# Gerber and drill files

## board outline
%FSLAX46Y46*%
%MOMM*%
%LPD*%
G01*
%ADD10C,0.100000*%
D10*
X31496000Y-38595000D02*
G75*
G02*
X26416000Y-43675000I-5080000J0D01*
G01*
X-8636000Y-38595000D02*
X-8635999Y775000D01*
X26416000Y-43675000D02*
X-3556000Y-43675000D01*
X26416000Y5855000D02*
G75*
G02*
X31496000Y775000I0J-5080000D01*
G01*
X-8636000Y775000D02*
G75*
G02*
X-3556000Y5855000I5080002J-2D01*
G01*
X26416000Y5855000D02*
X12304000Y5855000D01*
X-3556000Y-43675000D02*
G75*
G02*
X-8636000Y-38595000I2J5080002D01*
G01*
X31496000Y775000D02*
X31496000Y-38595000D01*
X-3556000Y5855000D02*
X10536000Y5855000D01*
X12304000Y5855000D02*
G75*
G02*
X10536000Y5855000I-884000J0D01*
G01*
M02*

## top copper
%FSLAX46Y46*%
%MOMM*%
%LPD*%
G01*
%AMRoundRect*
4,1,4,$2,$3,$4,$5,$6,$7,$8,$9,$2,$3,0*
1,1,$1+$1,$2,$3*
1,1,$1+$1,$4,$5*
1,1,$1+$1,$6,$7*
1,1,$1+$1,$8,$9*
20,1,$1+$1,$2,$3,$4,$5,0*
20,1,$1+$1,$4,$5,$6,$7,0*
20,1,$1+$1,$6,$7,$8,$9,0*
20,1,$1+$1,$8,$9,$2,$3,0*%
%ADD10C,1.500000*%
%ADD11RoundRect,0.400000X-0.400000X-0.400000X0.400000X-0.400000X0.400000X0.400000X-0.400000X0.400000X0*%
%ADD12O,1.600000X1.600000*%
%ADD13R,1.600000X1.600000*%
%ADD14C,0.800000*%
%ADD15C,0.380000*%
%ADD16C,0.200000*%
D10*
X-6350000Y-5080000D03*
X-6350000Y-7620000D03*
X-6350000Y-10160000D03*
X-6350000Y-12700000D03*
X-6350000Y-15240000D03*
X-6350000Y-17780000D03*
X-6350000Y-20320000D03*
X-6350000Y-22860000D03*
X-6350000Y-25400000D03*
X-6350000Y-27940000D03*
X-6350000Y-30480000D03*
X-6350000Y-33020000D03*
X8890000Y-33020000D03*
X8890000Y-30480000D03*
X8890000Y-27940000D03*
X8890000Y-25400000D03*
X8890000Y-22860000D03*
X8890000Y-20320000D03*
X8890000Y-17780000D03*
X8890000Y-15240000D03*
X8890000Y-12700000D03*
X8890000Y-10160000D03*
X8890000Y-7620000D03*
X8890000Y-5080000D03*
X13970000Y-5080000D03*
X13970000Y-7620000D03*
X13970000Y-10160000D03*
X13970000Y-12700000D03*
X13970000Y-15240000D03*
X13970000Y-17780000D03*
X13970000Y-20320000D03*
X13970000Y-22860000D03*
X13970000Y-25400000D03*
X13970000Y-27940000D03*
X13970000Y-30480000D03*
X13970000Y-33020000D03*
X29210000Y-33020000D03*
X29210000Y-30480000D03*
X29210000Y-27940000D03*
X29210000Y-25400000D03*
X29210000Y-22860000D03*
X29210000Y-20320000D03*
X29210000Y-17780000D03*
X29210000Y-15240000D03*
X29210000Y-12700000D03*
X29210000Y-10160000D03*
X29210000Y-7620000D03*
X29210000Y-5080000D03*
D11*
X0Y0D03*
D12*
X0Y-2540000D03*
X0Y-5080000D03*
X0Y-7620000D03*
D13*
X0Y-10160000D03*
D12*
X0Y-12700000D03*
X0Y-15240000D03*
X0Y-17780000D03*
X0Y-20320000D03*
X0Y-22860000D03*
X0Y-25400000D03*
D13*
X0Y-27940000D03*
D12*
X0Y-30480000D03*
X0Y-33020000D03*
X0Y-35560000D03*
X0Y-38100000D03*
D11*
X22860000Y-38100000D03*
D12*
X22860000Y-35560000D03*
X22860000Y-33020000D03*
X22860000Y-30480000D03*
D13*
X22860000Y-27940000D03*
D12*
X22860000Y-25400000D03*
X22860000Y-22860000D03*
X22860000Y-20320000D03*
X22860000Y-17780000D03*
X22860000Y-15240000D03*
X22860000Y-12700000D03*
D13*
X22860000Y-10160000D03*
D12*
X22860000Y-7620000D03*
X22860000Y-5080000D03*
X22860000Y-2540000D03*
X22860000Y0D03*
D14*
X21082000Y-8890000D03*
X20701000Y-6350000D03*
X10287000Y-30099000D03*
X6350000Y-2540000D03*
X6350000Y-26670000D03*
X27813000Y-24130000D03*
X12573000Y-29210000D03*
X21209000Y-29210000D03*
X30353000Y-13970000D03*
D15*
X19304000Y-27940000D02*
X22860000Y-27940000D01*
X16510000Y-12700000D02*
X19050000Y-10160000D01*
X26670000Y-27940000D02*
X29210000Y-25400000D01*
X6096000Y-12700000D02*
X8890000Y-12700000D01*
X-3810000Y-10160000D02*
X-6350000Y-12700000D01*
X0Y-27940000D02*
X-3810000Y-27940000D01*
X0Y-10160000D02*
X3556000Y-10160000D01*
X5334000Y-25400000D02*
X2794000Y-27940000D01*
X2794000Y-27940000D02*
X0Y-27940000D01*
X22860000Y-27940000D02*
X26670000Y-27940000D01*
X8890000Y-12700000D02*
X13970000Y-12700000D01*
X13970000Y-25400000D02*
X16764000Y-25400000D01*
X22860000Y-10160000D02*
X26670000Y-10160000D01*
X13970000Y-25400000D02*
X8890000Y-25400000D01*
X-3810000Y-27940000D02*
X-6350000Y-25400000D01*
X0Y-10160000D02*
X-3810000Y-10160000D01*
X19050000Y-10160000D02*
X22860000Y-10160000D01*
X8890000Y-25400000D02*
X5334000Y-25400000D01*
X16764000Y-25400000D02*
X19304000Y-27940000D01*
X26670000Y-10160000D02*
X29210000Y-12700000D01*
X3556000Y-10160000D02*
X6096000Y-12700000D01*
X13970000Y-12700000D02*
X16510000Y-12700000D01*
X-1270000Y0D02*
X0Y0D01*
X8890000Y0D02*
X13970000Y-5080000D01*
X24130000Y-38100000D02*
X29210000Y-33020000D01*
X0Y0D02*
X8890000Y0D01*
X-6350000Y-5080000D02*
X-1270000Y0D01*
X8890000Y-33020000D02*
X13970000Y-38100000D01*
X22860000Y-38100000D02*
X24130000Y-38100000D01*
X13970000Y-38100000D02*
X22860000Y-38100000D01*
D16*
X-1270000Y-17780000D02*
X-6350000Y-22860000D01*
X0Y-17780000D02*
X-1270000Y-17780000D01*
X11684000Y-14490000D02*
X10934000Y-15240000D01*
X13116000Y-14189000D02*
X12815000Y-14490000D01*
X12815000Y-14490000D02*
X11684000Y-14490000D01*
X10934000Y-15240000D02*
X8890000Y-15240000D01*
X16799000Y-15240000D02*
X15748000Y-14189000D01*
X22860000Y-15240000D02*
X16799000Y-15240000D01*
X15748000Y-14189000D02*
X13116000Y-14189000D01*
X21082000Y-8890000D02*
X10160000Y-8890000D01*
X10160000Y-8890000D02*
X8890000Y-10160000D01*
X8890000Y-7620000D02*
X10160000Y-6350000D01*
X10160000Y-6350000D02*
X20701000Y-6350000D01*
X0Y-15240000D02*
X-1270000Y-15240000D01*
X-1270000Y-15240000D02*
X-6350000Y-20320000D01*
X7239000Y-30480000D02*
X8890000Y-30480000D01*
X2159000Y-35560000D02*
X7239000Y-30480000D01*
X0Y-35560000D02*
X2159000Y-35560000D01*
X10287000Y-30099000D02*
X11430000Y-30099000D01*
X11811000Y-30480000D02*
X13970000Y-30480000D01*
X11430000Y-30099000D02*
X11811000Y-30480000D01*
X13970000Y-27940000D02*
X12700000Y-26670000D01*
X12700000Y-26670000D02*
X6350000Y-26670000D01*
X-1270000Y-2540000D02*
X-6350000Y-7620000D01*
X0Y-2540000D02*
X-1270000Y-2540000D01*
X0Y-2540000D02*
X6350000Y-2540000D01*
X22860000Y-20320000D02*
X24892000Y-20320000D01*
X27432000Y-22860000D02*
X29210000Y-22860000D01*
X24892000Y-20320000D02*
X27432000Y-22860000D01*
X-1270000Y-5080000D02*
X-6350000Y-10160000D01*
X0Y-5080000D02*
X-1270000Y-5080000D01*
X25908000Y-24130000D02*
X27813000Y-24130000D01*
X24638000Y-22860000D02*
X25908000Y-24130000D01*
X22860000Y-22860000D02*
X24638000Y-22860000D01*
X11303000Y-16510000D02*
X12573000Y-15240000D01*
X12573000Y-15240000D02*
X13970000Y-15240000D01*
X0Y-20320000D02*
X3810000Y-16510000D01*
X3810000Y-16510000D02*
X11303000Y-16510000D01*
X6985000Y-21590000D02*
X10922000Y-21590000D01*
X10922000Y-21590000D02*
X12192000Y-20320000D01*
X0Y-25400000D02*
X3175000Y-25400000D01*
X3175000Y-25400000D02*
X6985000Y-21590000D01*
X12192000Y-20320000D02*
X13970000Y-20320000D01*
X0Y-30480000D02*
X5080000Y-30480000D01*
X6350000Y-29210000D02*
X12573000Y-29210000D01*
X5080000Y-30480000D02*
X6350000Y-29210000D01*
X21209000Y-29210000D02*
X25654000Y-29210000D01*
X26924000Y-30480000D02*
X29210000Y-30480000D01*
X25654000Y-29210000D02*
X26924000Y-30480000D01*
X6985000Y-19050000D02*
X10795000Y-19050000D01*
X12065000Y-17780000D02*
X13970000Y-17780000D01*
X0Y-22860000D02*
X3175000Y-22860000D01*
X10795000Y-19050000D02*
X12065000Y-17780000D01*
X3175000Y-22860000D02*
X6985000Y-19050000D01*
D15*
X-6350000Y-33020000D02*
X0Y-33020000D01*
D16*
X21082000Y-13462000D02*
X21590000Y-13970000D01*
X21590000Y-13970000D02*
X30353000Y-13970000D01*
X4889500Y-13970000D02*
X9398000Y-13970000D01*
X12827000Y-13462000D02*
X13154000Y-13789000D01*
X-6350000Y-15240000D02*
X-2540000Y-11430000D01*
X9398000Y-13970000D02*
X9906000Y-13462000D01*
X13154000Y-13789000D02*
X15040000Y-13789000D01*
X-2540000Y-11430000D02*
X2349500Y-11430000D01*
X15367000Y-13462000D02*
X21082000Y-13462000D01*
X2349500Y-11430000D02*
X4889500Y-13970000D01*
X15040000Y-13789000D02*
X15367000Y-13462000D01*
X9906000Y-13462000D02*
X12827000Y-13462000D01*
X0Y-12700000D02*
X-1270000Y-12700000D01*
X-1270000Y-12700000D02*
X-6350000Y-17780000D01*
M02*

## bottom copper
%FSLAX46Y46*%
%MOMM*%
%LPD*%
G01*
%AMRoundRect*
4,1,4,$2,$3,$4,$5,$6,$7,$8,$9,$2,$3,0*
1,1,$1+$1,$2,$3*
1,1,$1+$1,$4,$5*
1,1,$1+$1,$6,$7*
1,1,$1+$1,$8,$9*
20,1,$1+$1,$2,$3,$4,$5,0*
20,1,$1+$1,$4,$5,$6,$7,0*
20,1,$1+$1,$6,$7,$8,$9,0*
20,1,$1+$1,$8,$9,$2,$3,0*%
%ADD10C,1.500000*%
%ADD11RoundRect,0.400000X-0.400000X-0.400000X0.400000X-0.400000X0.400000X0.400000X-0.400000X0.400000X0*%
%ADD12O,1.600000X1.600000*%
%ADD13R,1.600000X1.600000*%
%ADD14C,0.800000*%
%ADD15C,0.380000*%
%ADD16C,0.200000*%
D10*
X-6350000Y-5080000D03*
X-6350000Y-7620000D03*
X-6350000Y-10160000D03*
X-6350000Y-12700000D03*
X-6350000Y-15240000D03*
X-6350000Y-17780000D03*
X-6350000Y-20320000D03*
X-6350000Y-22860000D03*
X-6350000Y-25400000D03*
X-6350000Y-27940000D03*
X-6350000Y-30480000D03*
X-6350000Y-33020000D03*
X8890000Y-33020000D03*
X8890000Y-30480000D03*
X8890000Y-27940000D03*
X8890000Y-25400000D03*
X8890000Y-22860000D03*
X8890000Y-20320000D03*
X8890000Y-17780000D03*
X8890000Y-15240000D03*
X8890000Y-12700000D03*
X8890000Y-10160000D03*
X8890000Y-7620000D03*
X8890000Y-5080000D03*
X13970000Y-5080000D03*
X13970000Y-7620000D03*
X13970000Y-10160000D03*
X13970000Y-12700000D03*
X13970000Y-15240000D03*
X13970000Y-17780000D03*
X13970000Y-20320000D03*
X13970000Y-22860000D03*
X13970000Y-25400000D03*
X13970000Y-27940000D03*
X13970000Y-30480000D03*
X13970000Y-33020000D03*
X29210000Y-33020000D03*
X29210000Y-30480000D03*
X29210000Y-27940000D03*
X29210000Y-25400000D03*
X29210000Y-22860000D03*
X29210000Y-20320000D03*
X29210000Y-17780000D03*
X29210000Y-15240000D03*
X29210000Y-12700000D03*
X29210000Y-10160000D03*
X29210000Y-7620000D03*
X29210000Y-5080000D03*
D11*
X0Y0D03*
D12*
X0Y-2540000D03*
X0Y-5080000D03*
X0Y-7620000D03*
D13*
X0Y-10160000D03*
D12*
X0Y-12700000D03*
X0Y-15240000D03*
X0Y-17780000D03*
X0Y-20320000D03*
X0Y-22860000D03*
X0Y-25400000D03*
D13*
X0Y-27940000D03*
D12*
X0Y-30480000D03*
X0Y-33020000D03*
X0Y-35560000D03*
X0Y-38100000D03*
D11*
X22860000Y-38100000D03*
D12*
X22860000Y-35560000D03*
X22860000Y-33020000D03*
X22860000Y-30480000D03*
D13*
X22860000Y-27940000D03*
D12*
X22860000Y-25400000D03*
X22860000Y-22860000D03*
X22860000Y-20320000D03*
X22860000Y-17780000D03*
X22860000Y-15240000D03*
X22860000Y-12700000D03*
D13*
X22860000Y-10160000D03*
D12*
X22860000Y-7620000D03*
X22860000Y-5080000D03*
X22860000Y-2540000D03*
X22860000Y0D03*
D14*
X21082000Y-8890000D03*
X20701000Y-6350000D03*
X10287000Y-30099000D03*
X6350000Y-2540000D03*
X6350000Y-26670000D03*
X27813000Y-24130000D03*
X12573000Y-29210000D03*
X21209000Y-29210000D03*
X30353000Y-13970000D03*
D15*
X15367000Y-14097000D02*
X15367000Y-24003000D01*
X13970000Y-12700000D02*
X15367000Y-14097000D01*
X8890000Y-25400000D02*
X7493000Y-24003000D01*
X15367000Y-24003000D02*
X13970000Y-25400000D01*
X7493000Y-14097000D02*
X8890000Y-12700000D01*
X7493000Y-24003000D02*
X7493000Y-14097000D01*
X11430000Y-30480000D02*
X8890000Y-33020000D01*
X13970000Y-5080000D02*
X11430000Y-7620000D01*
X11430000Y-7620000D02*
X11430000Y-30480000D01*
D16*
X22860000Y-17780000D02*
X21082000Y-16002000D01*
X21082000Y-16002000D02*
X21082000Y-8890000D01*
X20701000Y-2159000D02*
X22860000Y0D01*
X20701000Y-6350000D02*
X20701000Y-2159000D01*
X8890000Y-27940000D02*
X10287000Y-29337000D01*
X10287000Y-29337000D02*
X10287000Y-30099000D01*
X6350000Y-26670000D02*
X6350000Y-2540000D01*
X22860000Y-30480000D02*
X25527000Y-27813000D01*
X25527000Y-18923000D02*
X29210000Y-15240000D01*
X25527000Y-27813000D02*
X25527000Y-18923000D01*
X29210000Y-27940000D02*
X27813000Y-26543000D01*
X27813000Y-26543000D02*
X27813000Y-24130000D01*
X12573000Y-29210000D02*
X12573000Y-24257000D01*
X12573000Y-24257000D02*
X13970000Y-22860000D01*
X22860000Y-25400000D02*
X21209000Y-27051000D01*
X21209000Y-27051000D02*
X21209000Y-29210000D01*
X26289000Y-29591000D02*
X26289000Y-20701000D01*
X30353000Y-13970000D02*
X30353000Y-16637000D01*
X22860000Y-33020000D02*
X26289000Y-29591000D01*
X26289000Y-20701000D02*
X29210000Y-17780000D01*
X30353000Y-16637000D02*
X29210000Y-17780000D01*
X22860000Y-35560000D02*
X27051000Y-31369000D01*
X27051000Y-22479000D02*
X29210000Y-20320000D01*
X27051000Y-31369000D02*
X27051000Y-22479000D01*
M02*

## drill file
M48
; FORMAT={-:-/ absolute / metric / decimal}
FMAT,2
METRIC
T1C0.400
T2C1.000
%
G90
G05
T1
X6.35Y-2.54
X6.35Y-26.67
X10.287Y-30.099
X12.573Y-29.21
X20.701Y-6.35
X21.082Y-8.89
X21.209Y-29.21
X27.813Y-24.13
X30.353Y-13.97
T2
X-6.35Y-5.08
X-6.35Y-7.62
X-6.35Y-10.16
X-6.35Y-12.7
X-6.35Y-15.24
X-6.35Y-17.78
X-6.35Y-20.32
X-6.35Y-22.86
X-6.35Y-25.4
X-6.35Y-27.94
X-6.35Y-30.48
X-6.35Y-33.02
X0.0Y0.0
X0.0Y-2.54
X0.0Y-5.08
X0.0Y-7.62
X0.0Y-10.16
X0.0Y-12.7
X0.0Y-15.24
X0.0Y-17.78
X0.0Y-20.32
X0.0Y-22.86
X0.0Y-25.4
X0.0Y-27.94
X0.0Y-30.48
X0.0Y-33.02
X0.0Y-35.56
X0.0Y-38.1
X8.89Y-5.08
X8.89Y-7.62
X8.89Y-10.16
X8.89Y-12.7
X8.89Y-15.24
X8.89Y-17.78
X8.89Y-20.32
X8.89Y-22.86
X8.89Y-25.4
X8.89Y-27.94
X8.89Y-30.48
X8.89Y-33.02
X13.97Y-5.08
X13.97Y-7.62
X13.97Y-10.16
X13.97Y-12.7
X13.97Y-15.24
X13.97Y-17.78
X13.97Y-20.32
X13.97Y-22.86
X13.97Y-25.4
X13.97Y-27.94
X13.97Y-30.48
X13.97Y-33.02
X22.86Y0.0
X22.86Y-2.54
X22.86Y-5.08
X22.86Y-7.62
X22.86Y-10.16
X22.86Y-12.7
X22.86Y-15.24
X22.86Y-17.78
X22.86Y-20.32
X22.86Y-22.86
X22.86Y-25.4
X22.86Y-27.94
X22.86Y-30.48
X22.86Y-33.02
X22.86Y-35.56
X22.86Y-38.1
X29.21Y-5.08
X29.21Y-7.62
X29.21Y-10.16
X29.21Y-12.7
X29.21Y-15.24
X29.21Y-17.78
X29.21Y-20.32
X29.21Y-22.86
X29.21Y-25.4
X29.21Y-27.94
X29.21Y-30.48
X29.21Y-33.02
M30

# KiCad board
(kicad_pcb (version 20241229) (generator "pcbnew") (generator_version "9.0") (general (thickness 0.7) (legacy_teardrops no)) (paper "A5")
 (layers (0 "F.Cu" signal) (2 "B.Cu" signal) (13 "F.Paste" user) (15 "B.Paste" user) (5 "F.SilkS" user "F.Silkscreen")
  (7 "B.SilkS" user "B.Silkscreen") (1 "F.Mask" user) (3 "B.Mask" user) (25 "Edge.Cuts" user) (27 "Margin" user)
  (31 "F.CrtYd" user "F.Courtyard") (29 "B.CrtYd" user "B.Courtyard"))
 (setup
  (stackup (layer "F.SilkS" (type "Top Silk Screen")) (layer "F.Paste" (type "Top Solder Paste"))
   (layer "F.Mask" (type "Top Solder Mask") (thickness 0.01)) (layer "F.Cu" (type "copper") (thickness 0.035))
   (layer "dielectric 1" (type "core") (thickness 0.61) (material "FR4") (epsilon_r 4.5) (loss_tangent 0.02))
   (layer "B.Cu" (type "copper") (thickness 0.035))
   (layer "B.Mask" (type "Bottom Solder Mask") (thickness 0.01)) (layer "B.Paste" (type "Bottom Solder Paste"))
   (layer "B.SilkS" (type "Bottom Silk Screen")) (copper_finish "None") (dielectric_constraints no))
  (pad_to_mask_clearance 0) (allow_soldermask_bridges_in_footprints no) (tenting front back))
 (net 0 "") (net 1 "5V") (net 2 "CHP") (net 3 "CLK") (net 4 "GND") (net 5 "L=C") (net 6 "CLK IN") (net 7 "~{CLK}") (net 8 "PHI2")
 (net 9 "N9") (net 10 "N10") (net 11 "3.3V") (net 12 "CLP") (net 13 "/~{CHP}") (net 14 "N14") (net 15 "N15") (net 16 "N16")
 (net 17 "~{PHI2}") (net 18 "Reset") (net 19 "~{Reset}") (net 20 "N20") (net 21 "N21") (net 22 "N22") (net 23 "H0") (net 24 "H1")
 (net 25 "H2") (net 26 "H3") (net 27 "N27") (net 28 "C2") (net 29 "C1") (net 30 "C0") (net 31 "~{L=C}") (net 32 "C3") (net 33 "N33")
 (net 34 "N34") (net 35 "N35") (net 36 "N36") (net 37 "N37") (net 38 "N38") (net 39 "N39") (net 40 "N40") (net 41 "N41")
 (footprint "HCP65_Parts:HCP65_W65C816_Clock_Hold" (layer "F.Cu") (at -6.35 5.08)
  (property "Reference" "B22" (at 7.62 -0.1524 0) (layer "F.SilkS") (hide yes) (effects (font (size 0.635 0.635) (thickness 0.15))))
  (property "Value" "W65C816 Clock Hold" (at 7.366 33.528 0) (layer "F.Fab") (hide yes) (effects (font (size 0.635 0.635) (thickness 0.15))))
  (pad "1" thru_hole circle (at 0 0) (size 1.5 1.5) (drill 1) (layers "*.Cu" "*.Mask") (remove_unused_layers no) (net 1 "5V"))
  (pad "2" thru_hole circle (at 0 2.54) (size 1.5 1.5) (drill 1) (layers "*.Cu" "*.Mask") (remove_unused_layers no) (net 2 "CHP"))
  (pad "3" thru_hole circle (at 0 5.08) (size 1.5 1.5) (drill 1) (layers "*.Cu" "*.Mask") (remove_unused_layers no) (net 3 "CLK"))
  (pad "4" thru_hole circle (at 0 7.62) (size 1.5 1.5) (drill 1) (layers "*.Cu" "*.Mask") (remove_unused_layers no) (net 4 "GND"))
  (pad "5" thru_hole circle (at 0 10.16) (size 1.5 1.5) (drill 1) (layers "*.Cu" "*.Mask") (remove_unused_layers no) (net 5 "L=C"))
  (pad "6" thru_hole circle (at 0 12.7) (size 1.5 1.5) (drill 1) (layers "*.Cu" "*.Mask") (remove_unused_layers no) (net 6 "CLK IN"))
  (pad "7" thru_hole circle (at 0 15.24) (size 1.5 1.5) (drill 1) (layers "*.Cu" "*.Mask") (remove_unused_layers no) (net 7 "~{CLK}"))
  (pad "8" thru_hole circle (at 0 17.78) (size 1.5 1.5) (drill 1) (layers "*.Cu" "*.Mask") (remove_unused_layers no) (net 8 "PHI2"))
  (pad "9" thru_hole circle (at 0 20.32) (size 1.5 1.5) (drill 1) (layers "*.Cu" "*.Mask") (remove_unused_layers no) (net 4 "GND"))
  (pad "10" thru_hole circle (at 0 22.86) (size 1.5 1.5) (drill 1) (layers "*.Cu" "*.Mask") (remove_unused_layers no) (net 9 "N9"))
  (pad "11" thru_hole circle (at 0 25.4) (size 1.5 1.5) (drill 1) (layers "*.Cu" "*.Mask") (remove_unused_layers no) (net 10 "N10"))
  (pad "12" thru_hole circle (at 0 27.94) (size 1.5 1.5) (drill 1) (layers "*.Cu" "*.Mask") (remove_unused_layers no) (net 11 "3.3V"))
  (pad "13" thru_hole circle (at 15.24 27.94) (size 1.5 1.5) (drill 1) (layers "*.Cu" "*.Mask") (remove_unused_layers no) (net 1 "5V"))
  (pad "14" thru_hole circle (at 15.24 25.4) (size 1.5 1.5) (drill 1) (layers "*.Cu" "*.Mask") (remove_unused_layers no) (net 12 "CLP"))
  (pad "15" thru_hole circle (at 15.24 22.86) (size 1.5 1.5) (drill 1) (layers "*.Cu" "*.Mask") (remove_unused_layers no) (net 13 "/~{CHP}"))
  (pad "16" thru_hole circle (at 15.24 20.32) (size 1.5 1.5) (drill 1) (layers "*.Cu" "*.Mask") (remove_unused_layers no) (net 4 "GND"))
  (pad "17" thru_hole circle (at 15.24 17.78) (size 1.5 1.5) (drill 1) (layers "*.Cu" "*.Mask") (remove_unused_layers no) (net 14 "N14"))
  (pad "18" thru_hole circle (at 15.24 15.24) (size 1.5 1.5) (drill 1) (layers "*.Cu" "*.Mask") (remove_unused_layers no) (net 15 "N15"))
  (pad "19" thru_hole circle (at 15.24 12.7) (size 1.5 1.5) (drill 1) (layers "*.Cu" "*.Mask") (remove_unused_layers no) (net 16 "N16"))
  (pad "20" thru_hole circle (at 15.24 10.16) (size 1.5 1.5) (drill 1) (layers "*.Cu" "*.Mask") (remove_unused_layers no) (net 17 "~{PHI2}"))
  (pad "21" thru_hole circle (at 15.24 7.62) (size 1.5 1.5) (drill 1) (layers "*.Cu" "*.Mask") (remove_unused_layers no) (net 4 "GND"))
  (pad "22" thru_hole circle (at 15.24 5.08) (size 1.5 1.5) (drill 1) (layers "*.Cu" "*.Mask") (remove_unused_layers no) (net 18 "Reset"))
  (pad "23" thru_hole circle (at 15.24 2.54) (size 1.5 1.5) (drill 1) (layers "*.Cu" "*.Mask") (remove_unused_layers no) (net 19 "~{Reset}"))
  (pad "24" thru_hole circle (at 15.24 0) (size 1.5 1.5) (drill 1) (layers "*.Cu" "*.Mask") (remove_unused_layers no) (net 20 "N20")))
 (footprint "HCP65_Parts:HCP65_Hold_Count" (layer "F.Cu") (at 13.97 5.08)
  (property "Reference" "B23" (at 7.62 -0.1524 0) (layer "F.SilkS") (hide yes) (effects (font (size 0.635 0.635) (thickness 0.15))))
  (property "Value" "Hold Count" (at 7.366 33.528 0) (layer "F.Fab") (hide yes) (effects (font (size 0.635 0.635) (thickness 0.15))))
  (pad "1" thru_hole circle (at 0 0) (size 1.5 1.5) (drill 1) (layers "*.Cu" "*.Mask") (remove_unused_layers no) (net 1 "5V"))
  (pad "2" thru_hole circle (at 0 2.54) (size 1.5 1.5) (drill 1) (layers "*.Cu" "*.Mask") (remove_unused_layers no) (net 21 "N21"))
  (pad "3" thru_hole circle (at 0 5.08) (size 1.5 1.5) (drill 1) (layers "*.Cu" "*.Mask") (remove_unused_layers no) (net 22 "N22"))
  (pad "4" thru_hole circle (at 0 7.62) (size 1.5 1.5) (drill 1) (layers "*.Cu" "*.Mask") (remove_unused_layers no) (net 4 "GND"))
  (pad "5" thru_hole circle (at 0 10.16) (size 1.5 1.5) (drill 1) (layers "*.Cu" "*.Mask") (remove_unused_layers no) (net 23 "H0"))
  (pad "6" thru_hole circle (at 0 12.7) (size 1.5 1.5) (drill 1) (layers "*.Cu" "*.Mask") (remove_unused_layers no) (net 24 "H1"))
  (pad "7" thru_hole circle (at 0 15.24) (size 1.5 1.5) (drill 1) (layers "*.Cu" "*.Mask") (remove_unused_layers no) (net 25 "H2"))
  (pad "8" thru_hole circle (at 0 17.78) (size 1.5 1.5) (drill 1) (layers "*.Cu" "*.Mask") (remove_unused_layers no) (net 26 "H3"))
  (pad "9" thru_hole circle (at 0 20.32) (size 1.5 1.5) (drill 1) (layers "*.Cu" "*.Mask") (remove_unused_layers no) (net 4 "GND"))
  (pad "10" thru_hole circle (at 0 22.86) (size 1.5 1.5) (drill 1) (layers "*.Cu" "*.Mask") (remove_unused_layers no) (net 2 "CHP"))
  (pad "11" thru_hole circle (at 0 25.4) (size 1.5 1.5) (drill 1) (layers "*.Cu" "*.Mask") (remove_unused_layers no) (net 13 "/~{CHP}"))
  (pad "12" thru_hole circle (at 0 27.94) (size 1.5 1.5) (drill 1) (layers "*.Cu" "*.Mask") (remove_unused_layers no) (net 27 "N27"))
  (pad "13" thru_hole circle (at 15.24 27.94) (size 1.5 1.5) (drill 1) (layers "*.Cu" "*.Mask") (remove_unused_layers no) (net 1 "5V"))
  (pad "14" thru_hole circle (at 15.24 25.4) (size 1.5 1.5) (drill 1) (layers "*.Cu" "*.Mask") (remove_unused_layers no) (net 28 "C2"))
  (pad "15" thru_hole circle (at 15.24 22.86) (size 1.5 1.5) (drill 1) (layers "*.Cu" "*.Mask") (remove_unused_layers no) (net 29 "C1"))
  (pad "16" thru_hole circle (at 15.24 20.32) (size 1.5 1.5) (drill 1) (layers "*.Cu" "*.Mask") (remove_unused_layers no) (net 4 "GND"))
  (pad "17" thru_hole circle (at 15.24 17.78) (size 1.5 1.5) (drill 1) (layers "*.Cu" "*.Mask") (remove_unused_layers no) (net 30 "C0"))
  (pad "18" thru_hole circle (at 15.24 15.24) (size 1.5 1.5) (drill 1) (layers "*.Cu" "*.Mask") (remove_unused_layers no) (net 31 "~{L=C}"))
  (pad "19" thru_hole circle (at 15.24 12.7) (size 1.5 1.5) (drill 1) (layers "*.Cu" "*.Mask") (remove_unused_layers no) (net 5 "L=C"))
  (pad "20" thru_hole circle (at 15.24 10.16) (size 1.5 1.5) (drill 1) (layers "*.Cu" "*.Mask") (remove_unused_layers no) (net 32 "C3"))
  (pad "21" thru_hole circle (at 15.24 7.62) (size 1.5 1.5) (drill 1) (layers "*.Cu" "*.Mask") (remove_unused_layers no) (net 4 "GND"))
  (pad "22" thru_hole circle (at 15.24 5.08) (size 1.5 1.5) (drill 1) (layers "*.Cu" "*.Mask") (remove_unused_layers no) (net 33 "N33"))
  (pad "23" thru_hole circle (at 15.24 2.54) (size 1.5 1.5) (drill 1) (layers "*.Cu" "*.Mask") (remove_unused_layers no) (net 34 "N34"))
  (pad "24" thru_hole circle (at 15.24 0) (size 1.5 1.5) (drill 1) (layers "*.Cu" "*.Mask") (remove_unused_layers no) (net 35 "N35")))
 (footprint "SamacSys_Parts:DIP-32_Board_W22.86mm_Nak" (layer "F.Cu") (at 0 0)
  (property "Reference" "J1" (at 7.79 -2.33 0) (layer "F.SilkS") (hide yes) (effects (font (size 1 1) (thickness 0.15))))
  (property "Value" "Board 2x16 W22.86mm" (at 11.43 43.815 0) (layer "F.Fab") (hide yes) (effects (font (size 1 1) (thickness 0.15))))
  (pad "1" thru_hole roundrect (at 0 0) (size 1.6 1.6) (drill 1) (layers "*.Cu" "*.Mask") (remove_unused_layers no) (roundrect_rratio 0.25)
   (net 1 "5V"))
  (pad "2" thru_hole oval (at 0 2.54) (size 1.6 1.6) (drill 1) (layers "*.Cu" "*.Mask") (remove_unused_layers no) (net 2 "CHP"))
  (pad "3" thru_hole oval (at 0 5.08) (size 1.6 1.6) (drill 1) (layers "*.Cu" "*.Mask") (remove_unused_layers no) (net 3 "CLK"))
  (pad "4" thru_hole oval (at 0 7.62) (size 1.6 1.6) (drill 1) (layers "*.Cu" "*.Mask") (remove_unused_layers no) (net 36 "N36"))
  (pad "5" thru_hole rect (at 0 10.16) (size 1.6 1.6) (drill 1) (layers "*.Cu" "*.Mask") (remove_unused_layers no) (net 4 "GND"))
  (pad "6" thru_hole oval (at 0 12.7) (size 1.6 1.6) (drill 1) (layers "*.Cu" "*.Mask") (remove_unused_layers no) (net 6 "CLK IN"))
  (pad "7" thru_hole oval (at 0 15.24) (size 1.6 1.6) (drill 1) (layers "*.Cu" "*.Mask") (remove_unused_layers no) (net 7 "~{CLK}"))
  (pad "8" thru_hole oval (at 0 17.78) (size 1.6 1.6) (drill 1) (layers "*.Cu" "*.Mask") (remove_unused_layers no) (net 8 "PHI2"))
  (pad "9" thru_hole oval (at 0 20.32) (size 1.6 1.6) (drill 1) (layers "*.Cu" "*.Mask") (remove_unused_layers no) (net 23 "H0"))
  (pad "10" thru_hole oval (at 0 22.86) (size 1.6 1.6) (drill 1) (layers "*.Cu" "*.Mask") (remove_unused_layers no) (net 24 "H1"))
  (pad "11" thru_hole oval (at 0 25.4) (size 1.6 1.6) (drill 1) (layers "*.Cu" "*.Mask") (remove_unused_layers no) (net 25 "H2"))
  (pad "12" thru_hole rect (at 0 27.94) (size 1.6 1.6) (drill 1) (layers "*.Cu" "*.Mask") (remove_unused_layers no) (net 4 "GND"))
  (pad "13" thru_hole oval (at 0 30.48) (size 1.6 1.6) (drill 1) (layers "*.Cu" "*.Mask") (remove_unused_layers no) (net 26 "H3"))
  (pad "14" thru_hole oval (at 0 33.02) (size 1.6 1.6) (drill 1) (layers "*.Cu" "*.Mask") (remove_unused_layers no) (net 11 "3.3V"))
  (pad "15" thru_hole oval (at 0 35.56) (size 1.6 1.6) (drill 1) (layers "*.Cu" "*.Mask") (remove_unused_layers no) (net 12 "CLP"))
  (pad "16" thru_hole oval (at 0 38.1) (size 1.6 1.6) (drill 1) (layers "*.Cu" "*.Mask") (remove_unused_layers no) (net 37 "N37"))
  (pad "17" thru_hole roundrect (at 22.86 38.1) (size 1.6 1.6) (drill 1) (layers "*.Cu" "*.Mask") (remove_unused_layers no)
   (roundrect_rratio 0.25) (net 1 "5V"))
  (pad "18" thru_hole oval (at 22.86 35.56) (size 1.6 1.6) (drill 1) (layers "*.Cu" "*.Mask") (remove_unused_layers no) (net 31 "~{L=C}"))
  (pad "19" thru_hole oval (at 22.86 33.02) (size 1.6 1.6) (drill 1) (layers "*.Cu" "*.Mask") (remove_unused_layers no) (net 5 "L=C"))
  (pad "20" thru_hole oval (at 22.86 30.48) (size 1.6 1.6) (drill 1) (layers "*.Cu" "*.Mask") (remove_unused_layers no) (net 32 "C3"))
  (pad "21" thru_hole rect (at 22.86 27.94) (size 1.6 1.6) (drill 1) (layers "*.Cu" "*.Mask") (remove_unused_layers no) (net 4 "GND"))
  (pad "22" thru_hole oval (at 22.86 25.4) (size 1.6 1.6) (drill 1) (layers "*.Cu" "*.Mask") (remove_unused_layers no) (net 28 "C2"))
  (pad "23" thru_hole oval (at 22.86 22.86) (size 1.6 1.6) (drill 1) (layers "*.Cu" "*.Mask") (remove_unused_layers no) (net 29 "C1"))
  (pad "24" thru_hole oval (at 22.86 20.32) (size 1.6 1.6) (drill 1) (layers "*.Cu" "*.Mask") (remove_unused_layers no) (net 30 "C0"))
  (pad "25" thru_hole oval (at 22.86 17.78) (size 1.6 1.6) (drill 1) (layers "*.Cu" "*.Mask") (remove_unused_layers no) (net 18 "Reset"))
  (pad "26" thru_hole oval (at 22.86 15.24) (size 1.6 1.6) (drill 1) (layers "*.Cu" "*.Mask") (remove_unused_layers no) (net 17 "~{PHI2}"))
  (pad "27" thru_hole oval (at 22.86 12.7) (size 1.6 1.6) (drill 1) (layers "*.Cu" "*.Mask") (remove_unused_layers no) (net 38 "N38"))
  (pad "28" thru_hole rect (at 22.86 10.16) (size 1.6 1.6) (drill 1) (layers "*.Cu" "*.Mask") (remove_unused_layers no) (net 4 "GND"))
  (pad "29" thru_hole oval (at 22.86 7.62) (size 1.6 1.6) (drill 1) (layers "*.Cu" "*.Mask") (remove_unused_layers no) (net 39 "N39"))
  (pad "30" thru_hole oval (at 22.86 5.08) (size 1.6 1.6) (drill 1) (layers "*.Cu" "*.Mask") (remove_unused_layers no) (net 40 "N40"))
  (pad "31" thru_hole oval (at 22.86 2.54) (size 1.6 1.6) (drill 1) (layers "*.Cu" "*.Mask") (remove_unused_layers no) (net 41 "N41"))
  (pad "32" thru_hole oval (at 22.86 0) (size 1.6 1.6) (drill 1) (layers "*.Cu" "*.Mask") (remove_unused_layers no) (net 19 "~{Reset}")))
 (gr_arc (start 31.496 38.595) (mid 30.008102 42.187102) (end 26.416 43.675) (stroke (width 0.1) (type default)) (layer "Edge.Cuts"))
 (gr_line (start -8.636 38.595) (end -8.635999 -0.775) (stroke (width 0.1) (type default)) (layer "Edge.Cuts"))
 (gr_line (start 26.416 43.675) (end -3.556 43.675) (stroke (width 0.1) (type default)) (layer "Edge.Cuts"))
 (gr_arc (start 26.416 -5.855) (mid 30.008102 -4.367102) (end 31.496 -0.775) (stroke (width 0.1) (type default)) (layer "Edge.Cuts"))
 (gr_arc (start -8.636 -0.775) (mid -7.148102 -4.367102) (end -3.556 -5.855) (stroke (width 0.1) (type default)) (layer "Edge.Cuts"))
 (gr_line (start 26.416 -5.855) (end 12.304 -5.855) (stroke (width 0.1) (type solid)) (layer "Edge.Cuts"))
 (gr_arc (start -3.556 43.675) (mid -7.148102 42.187102) (end -8.636 38.595) (stroke (width 0.1) (type default)) (layer "Edge.Cuts"))
 (gr_line (start 31.496 -0.775) (end 31.496 38.595) (stroke (width 0.1) (type default)) (layer "Edge.Cuts"))
 (gr_line (start -3.556 -5.855) (end 10.536 -5.855) (stroke (width 0.1) (type default)) (layer "Edge.Cuts"))
 (gr_arc (start 12.304 -5.855) (mid 11.42 -4.971) (end 10.536 -5.855) (stroke (width 0.1) (type solid)) (layer "Edge.Cuts"))
 (segment (start 19.304 27.94) (end 22.86 27.94) (width 0.38) (layer "F.Cu") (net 4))
 (segment (start 16.51 12.7) (end 19.05 10.16) (width 0.38) (layer "F.Cu") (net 4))
 (segment (start 26.67 27.94) (end 29.21 25.4) (width 0.38) (layer "F.Cu") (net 4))
 (segment (start 6.096 12.7) (end 8.89 12.7) (width 0.38) (layer "F.Cu") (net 4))
 (segment (start -3.81 10.16) (end -6.35 12.7) (width 0.38) (layer "F.Cu") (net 4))
 (segment (start 0 27.94) (end -3.81 27.94) (width 0.38) (layer "F.Cu") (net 4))
 (segment (start 0 10.16) (end 3.556 10.16) (width 0.38) (layer "F.Cu") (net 4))
 (segment (start 5.334 25.4) (end 2.794 27.94) (width 0.38) (layer "F.Cu") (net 4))
 (segment (start 2.794 27.94) (end 0 27.94) (width 0.38) (layer "F.Cu") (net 4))
 (segment (start 22.86 27.94) (end 26.67 27.94) (width 0.38) (layer "F.Cu") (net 4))
 (segment (start 8.89 12.7) (end 13.97 12.7) (width 0.38) (layer "F.Cu") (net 4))
 (segment (start 13.97 25.4) (end 16.764 25.4) (width 0.38) (layer "F.Cu") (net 4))
 (segment (start 22.86 10.16) (end 26.67 10.16) (width 0.38) (layer "F.Cu") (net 4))
 (segment (start 13.97 25.4) (end 8.89 25.4) (width 0.38) (layer "F.Cu") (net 4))
 (segment (start -3.81 27.94) (end -6.35 25.4) (width 0.38) (layer "F.Cu") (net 4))
 (segment (start 0 10.16) (end -3.81 10.16) (width 0.38) (layer "F.Cu") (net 4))
 (segment (start 19.05 10.16) (end 22.86 10.16) (width 0.38) (layer "F.Cu") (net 4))
 (segment (start 8.89 25.4) (end 5.334 25.4) (width 0.38) (layer "F.Cu") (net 4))
 (segment (start 16.764 25.4) (end 19.304 27.94) (width 0.38) (layer "F.Cu") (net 4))
 (segment (start 26.67 10.16) (end 29.21 12.7) (width 0.38) (layer "F.Cu") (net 4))
 (segment (start 3.556 10.16) (end 6.096 12.7) (width 0.38) (layer "F.Cu") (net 4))
 (segment (start 13.97 12.7) (end 16.51 12.7) (width 0.38) (layer "F.Cu") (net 4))
 (segment (start 15.367 14.097) (end 15.367 24.003) (width 0.38) (layer "B.Cu") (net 4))
 (segment (start 13.97 12.7) (end 15.367 14.097) (width 0.38) (layer "B.Cu") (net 4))
 (segment (start 8.89 25.4) (end 7.493 24.003) (width 0.38) (layer "B.Cu") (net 4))
 (segment (start 15.367 24.003) (end 13.97 25.4) (width 0.38) (layer "B.Cu") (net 4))
 (segment (start 7.493 14.097) (end 8.89 12.7) (width 0.38) (layer "B.Cu") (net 4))
 (segment (start 7.493 24.003) (end 7.493 14.097) (width 0.38) (layer "B.Cu") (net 4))
 (segment (start -1.27 0) (end 0 0) (width 0.38) (layer "F.Cu") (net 1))
 (segment (start 8.89 0) (end 13.97 5.08) (width 0.38) (layer "F.Cu") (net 1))
 (segment (start 24.13 38.1) (end 29.21 33.02) (width 0.38) (layer "F.Cu") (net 1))
 (segment (start 0 0) (end 8.89 0) (width 0.38) (layer "F.Cu") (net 1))
 (segment (start -6.35 5.08) (end -1.27 0) (width 0.38) (layer "F.Cu") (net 1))
 (segment (start 8.89 33.02) (end 13.97 38.1) (width 0.38) (layer "F.Cu") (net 1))
 (segment (start 22.86 38.1) (end 24.13 38.1) (width 0.38) (layer "F.Cu") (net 1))
 (segment (start 13.97 38.1) (end 22.86 38.1) (width 0.38) (layer "F.Cu") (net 1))
 (segment (start 11.43 30.48) (end 8.89 33.02) (width 0.38) (layer "B.Cu") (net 1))
 (segment (start 13.97 5.08) (end 11.43 7.62) (width 0.38) (layer "B.Cu") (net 1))
 (segment (start 11.43 7.62) (end 11.43 30.48) (width 0.38) (layer "B.Cu") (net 1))
 (segment (start -1.27 17.78) (end -6.35 22.86) (width 0.2) (layer "F.Cu") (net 8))
 (segment (start 0 17.78) (end -1.27 17.78) (width 0.2) (layer "F.Cu") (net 8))
 (segment (start 11.684 14.49) (end 10.934 15.24) (width 0.2) (layer "F.Cu") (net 17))
 (segment (start 13.116 14.189) (end 12.815 14.49) (width 0.2) (layer "F.Cu") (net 17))
 (segment (start 12.815 14.49) (end 11.684 14.49) (width 0.2) (layer "F.Cu") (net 17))
 (segment (start 10.934 15.24) (end 8.89 15.24) (width 0.2) (layer "F.Cu") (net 17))
 (segment (start 16.799 15.24) (end 15.748 14.189) (width 0.2) (layer "F.Cu") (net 17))
 (segment (start 22.86 15.24) (end 16.799 15.24) (width 0.2) (layer "F.Cu") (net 17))
 (segment (start 15.748 14.189) (end 13.116 14.189) (width 0.2) (layer "F.Cu") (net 17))
 (segment (start 21.082 8.89) (end 10.16 8.89) (width 0.2) (layer "F.Cu") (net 18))
 (segment (start 10.16 8.89) (end 8.89 10.16) (width 0.2) (layer "F.Cu") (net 18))
 (via (at 21.082 8.89) (size 0.8) (drill 0.4) (layers "F.Cu" "B.Cu") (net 18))
 (segment (start 22.86 17.78) (end 21.082 16.002) (width 0.2) (layer "B.Cu") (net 18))
 (segment (start 21.082 16.002) (end 21.082 8.89) (width 0.2) (layer "B.Cu") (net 18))
 (segment (start 8.89 7.62) (end 10.16 6.35) (width 0.2) (layer "F.Cu") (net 19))
 (segment (start 10.16 6.35) (end 20.701 6.35) (width 0.2) (layer "F.Cu") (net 19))
 (via (at 20.701 6.35) (size 0.8) (drill 0.4) (layers "F.Cu" "B.Cu") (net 19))
 (segment (start 20.701 2.159) (end 22.86 0) (width 0.2) (layer "B.Cu") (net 19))
 (segment (start 20.701 6.35) (end 20.701 2.159) (width 0.2) (layer "B.Cu") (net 19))
 (segment (start 0 15.24) (end -1.27 15.24) (width 0.2) (layer "F.Cu") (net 7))
 (segment (start -1.27 15.24) (end -6.35 20.32) (width 0.2) (layer "F.Cu") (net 7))
 (segment (start 7.239 30.48) (end 8.89 30.48) (width 0.2) (layer "F.Cu") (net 12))
 (segment (start 2.159 35.56) (end 7.239 30.48) (width 0.2) (layer "F.Cu") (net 12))
 (segment (start 0 35.56) (end 2.159 35.56) (width 0.2) (layer "F.Cu") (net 12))
 (segment (start 10.287 30.099) (end 11.43 30.099) (width 0.2) (layer "F.Cu") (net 13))
 (segment (start 11.811 30.48) (end 13.97 30.48) (width 0.2) (layer "F.Cu") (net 13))
 (segment (start 11.43 30.099) (end 11.811 30.48) (width 0.2) (layer "F.Cu") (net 13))
 (via (at 10.287 30.099) (size 0.8) (drill 0.4) (layers "F.Cu" "B.Cu") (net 13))
 (segment (start 8.89 27.94) (end 10.287 29.337) (width 0.2) (layer "B.Cu") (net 13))
 (segment (start 10.287 29.337) (end 10.287 30.099) (width 0.2) (layer "B.Cu") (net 13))
 (segment (start 13.97 27.94) (end 12.7 26.67) (width 0.2) (layer "F.Cu") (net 2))
 (segment (start 12.7 26.67) (end 6.35 26.67) (width 0.2) (layer "F.Cu") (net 2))
 (segment (start -1.27 2.54) (end -6.35 7.62) (width 0.2) (layer "F.Cu") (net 2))
 (segment (start 0 2.54) (end -1.27 2.54) (width 0.2) (layer "F.Cu") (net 2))
 (segment (start 0 2.54) (end 6.35 2.54) (width 0.2) (layer "F.Cu") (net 2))
 (via (at 6.35 2.54) (size 0.8) (drill 0.4) (layers "F.Cu" "B.Cu") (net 2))
 (via (at 6.35 26.67) (size 0.8) (drill 0.4) (layers "F.Cu" "B.Cu") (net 2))
 (segment (start 6.35 26.67) (end 6.35 2.54) (width 0.2) (layer "B.Cu") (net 2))
 (segment (start 22.86 20.32) (end 24.892 20.32) (width 0.2) (layer "F.Cu") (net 30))
 (segment (start 27.432 22.86) (end 29.21 22.86) (width 0.2) (layer "F.Cu") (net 30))
 (segment (start 24.892 20.32) (end 27.432 22.86) (width 0.2) (layer "F.Cu") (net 30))
 (segment (start -1.27 5.08) (end -6.35 10.16) (width 0.2) (layer "F.Cu") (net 3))
 (segment (start 0 5.08) (end -1.27 5.08) (width 0.2) (layer "F.Cu") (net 3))
 (segment (start 22.86 30.48) (end 25.527 27.813) (width 0.2) (layer "B.Cu") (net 32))
 (segment (start 25.527 18.923) (end 29.21 15.24) (width 0.2) (layer "B.Cu") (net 32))
 (segment (start 25.527 27.813) (end 25.527 18.923) (width 0.2) (layer "B.Cu") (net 32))
 (segment (start 25.908 24.13) (end 27.813 24.13) (width 0.2) (layer "F.Cu") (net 29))
 (segment (start 24.638 22.86) (end 25.908 24.13) (width 0.2) (layer "F.Cu") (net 29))
 (segment (start 22.86 22.86) (end 24.638 22.86) (width 0.2) (layer "F.Cu") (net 29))
 (via (at 27.813 24.13) (size 0.8) (drill 0.4) (layers "F.Cu" "B.Cu") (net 29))
 (segment (start 29.21 27.94) (end 27.813 26.543) (width 0.2) (layer "B.Cu") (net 29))
 (segment (start 27.813 26.543) (end 27.813 24.13) (width 0.2) (layer "B.Cu") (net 29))
 (segment (start 11.303 16.51) (end 12.573 15.24) (width 0.2) (layer "F.Cu") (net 23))
 (segment (start 12.573 15.24) (end 13.97 15.24) (width 0.2) (layer "F.Cu") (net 23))
 (segment (start 0 20.32) (end 3.81 16.51) (width 0.2) (layer "F.Cu") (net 23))
 (segment (start 3.81 16.51) (end 11.303 16.51) (width 0.2) (layer "F.Cu") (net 23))
 (segment (start 6.985 21.59) (end 10.922 21.59) (width 0.2) (layer "F.Cu") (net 25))
 (segment (start 10.922 21.59) (end 12.192 20.32) (width 0.2) (layer "F.Cu") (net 25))
 (segment (start 0 25.4) (end 3.175 25.4) (width 0.2) (layer "F.Cu") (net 25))
 (segment (start 3.175 25.4) (end 6.985 21.59) (width 0.2) (layer "F.Cu") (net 25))
 (segment (start 12.192 20.32) (end 13.97 20.32) (width 0.2) (layer "F.Cu") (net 25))
 (segment (start 0 30.48) (end 5.08 30.48) (width 0.2) (layer "F.Cu") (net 26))
 (segment (start 6.35 29.21) (end 12.573 29.21) (width 0.2) (layer "F.Cu") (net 26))
 (segment (start 5.08 30.48) (end 6.35 29.21) (width 0.2) (layer "F.Cu") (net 26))
 (via (at 12.573 29.21) (size 0.8) (drill 0.4) (layers "F.Cu" "B.Cu") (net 26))
 (segment (start 12.573 29.21) (end 12.573 24.257) (width 0.2) (layer "B.Cu") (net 26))
 (segment (start 12.573 24.257) (end 13.97 22.86) (width 0.2) (layer "B.Cu") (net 26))
 (segment (start 21.209 29.21) (end 25.654 29.21) (width 0.2) (layer "F.Cu") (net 28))
 (segment (start 26.924 30.48) (end 29.21 30.48) (width 0.2) (layer "F.Cu") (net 28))
 (segment (start 25.654 29.21) (end 26.924 30.48) (width 0.2) (layer "F.Cu") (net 28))
 (via (at 21.209 29.21) (size 0.8) (drill 0.4) (layers "F.Cu" "B.Cu") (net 28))
 (segment (start 22.86 25.4) (end 21.209 27.051) (width 0.2) (layer "B.Cu") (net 28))
 (segment (start 21.209 27.051) (end 21.209 29.21) (width 0.2) (layer "B.Cu") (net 28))
 (segment (start 6.985 19.05) (end 10.795 19.05) (width 0.2) (layer "F.Cu") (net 24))
 (segment (start 12.065 17.78) (end 13.97 17.78) (width 0.2) (layer "F.Cu") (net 24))
 (segment (start 0 22.86) (end 3.175 22.86) (width 0.2) (layer "F.Cu") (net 24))
 (segment (start 10.795 19.05) (end 12.065 17.78) (width 0.2) (layer "F.Cu") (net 24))
 (segment (start 3.175 22.86) (end 6.985 19.05) (width 0.2) (layer "F.Cu") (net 24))
 (segment (start -6.35 33.02) (end 0 33.02) (width 0.38) (layer "F.Cu") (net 11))
 (segment (start 21.082 13.462) (end 21.59 13.97) (width 0.2) (layer "F.Cu") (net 5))
 (segment (start 21.59 13.97) (end 30.353 13.97) (width 0.2) (layer "F.Cu") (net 5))
 (segment (start 4.8895 13.97) (end 9.398 13.97) (width 0.2) (layer "F.Cu") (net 5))
 (segment (start 12.827 13.462) (end 13.154 13.789) (width 0.2) (layer "F.Cu") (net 5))
 (segment (start -6.35 15.24) (end -2.54 11.43) (width 0.2) (layer "F.Cu") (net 5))
 (segment (start 9.398 13.97) (end 9.906 13.462) (width 0.2) (layer "F.Cu") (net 5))
 (segment (start 13.154 13.789) (end 15.04 13.789) (width 0.2) (layer "F.Cu") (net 5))
 (segment (start -2.54 11.43) (end 2.3495 11.43) (width 0.2) (layer "F.Cu") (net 5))
 (segment (start 15.367 13.462) (end 21.082 13.462) (width 0.2) (layer "F.Cu") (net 5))
 (segment (start 2.3495 11.43) (end 4.8895 13.97) (width 0.2) (layer "F.Cu") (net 5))
 (segment (start 15.04 13.789) (end 15.367 13.462) (width 0.2) (layer "F.Cu") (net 5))
 (segment (start 9.906 13.462) (end 12.827 13.462) (width 0.2) (layer "F.Cu") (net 5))
 (via (at 30.353 13.97) (size 0.8) (drill 0.4) (layers "F.Cu" "B.Cu") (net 5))
 (segment (start 26.289 29.591) (end 26.289 20.701) (width 0.2) (layer "B.Cu") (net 5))
 (segment (start 30.353 13.97) (end 30.353 16.637) (width 0.2) (layer "B.Cu") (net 5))
 (segment (start 22.86 33.02) (end 26.289 29.591) (width 0.2) (layer "B.Cu") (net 5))
 (segment (start 26.289 20.701) (end 29.21 17.78) (width 0.2) (layer "B.Cu") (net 5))
 (segment (start 30.353 16.637) (end 29.21 17.78) (width 0.2) (layer "B.Cu") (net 5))
 (segment (start 22.86 35.56) (end 27.051 31.369) (width 0.2) (layer "B.Cu") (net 31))
 (segment (start 27.051 22.479) (end 29.21 20.32) (width 0.2) (layer "B.Cu") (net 31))
 (segment (start 27.051 31.369) (end 27.051 22.479) (width 0.2) (layer "B.Cu") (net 31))
 (segment (start 0 12.7) (end -1.27 12.7) (width 0.2) (layer "F.Cu") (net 6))
 (segment (start -1.27 12.7) (end -6.35 17.78) (width 0.2) (layer "F.Cu") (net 6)))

